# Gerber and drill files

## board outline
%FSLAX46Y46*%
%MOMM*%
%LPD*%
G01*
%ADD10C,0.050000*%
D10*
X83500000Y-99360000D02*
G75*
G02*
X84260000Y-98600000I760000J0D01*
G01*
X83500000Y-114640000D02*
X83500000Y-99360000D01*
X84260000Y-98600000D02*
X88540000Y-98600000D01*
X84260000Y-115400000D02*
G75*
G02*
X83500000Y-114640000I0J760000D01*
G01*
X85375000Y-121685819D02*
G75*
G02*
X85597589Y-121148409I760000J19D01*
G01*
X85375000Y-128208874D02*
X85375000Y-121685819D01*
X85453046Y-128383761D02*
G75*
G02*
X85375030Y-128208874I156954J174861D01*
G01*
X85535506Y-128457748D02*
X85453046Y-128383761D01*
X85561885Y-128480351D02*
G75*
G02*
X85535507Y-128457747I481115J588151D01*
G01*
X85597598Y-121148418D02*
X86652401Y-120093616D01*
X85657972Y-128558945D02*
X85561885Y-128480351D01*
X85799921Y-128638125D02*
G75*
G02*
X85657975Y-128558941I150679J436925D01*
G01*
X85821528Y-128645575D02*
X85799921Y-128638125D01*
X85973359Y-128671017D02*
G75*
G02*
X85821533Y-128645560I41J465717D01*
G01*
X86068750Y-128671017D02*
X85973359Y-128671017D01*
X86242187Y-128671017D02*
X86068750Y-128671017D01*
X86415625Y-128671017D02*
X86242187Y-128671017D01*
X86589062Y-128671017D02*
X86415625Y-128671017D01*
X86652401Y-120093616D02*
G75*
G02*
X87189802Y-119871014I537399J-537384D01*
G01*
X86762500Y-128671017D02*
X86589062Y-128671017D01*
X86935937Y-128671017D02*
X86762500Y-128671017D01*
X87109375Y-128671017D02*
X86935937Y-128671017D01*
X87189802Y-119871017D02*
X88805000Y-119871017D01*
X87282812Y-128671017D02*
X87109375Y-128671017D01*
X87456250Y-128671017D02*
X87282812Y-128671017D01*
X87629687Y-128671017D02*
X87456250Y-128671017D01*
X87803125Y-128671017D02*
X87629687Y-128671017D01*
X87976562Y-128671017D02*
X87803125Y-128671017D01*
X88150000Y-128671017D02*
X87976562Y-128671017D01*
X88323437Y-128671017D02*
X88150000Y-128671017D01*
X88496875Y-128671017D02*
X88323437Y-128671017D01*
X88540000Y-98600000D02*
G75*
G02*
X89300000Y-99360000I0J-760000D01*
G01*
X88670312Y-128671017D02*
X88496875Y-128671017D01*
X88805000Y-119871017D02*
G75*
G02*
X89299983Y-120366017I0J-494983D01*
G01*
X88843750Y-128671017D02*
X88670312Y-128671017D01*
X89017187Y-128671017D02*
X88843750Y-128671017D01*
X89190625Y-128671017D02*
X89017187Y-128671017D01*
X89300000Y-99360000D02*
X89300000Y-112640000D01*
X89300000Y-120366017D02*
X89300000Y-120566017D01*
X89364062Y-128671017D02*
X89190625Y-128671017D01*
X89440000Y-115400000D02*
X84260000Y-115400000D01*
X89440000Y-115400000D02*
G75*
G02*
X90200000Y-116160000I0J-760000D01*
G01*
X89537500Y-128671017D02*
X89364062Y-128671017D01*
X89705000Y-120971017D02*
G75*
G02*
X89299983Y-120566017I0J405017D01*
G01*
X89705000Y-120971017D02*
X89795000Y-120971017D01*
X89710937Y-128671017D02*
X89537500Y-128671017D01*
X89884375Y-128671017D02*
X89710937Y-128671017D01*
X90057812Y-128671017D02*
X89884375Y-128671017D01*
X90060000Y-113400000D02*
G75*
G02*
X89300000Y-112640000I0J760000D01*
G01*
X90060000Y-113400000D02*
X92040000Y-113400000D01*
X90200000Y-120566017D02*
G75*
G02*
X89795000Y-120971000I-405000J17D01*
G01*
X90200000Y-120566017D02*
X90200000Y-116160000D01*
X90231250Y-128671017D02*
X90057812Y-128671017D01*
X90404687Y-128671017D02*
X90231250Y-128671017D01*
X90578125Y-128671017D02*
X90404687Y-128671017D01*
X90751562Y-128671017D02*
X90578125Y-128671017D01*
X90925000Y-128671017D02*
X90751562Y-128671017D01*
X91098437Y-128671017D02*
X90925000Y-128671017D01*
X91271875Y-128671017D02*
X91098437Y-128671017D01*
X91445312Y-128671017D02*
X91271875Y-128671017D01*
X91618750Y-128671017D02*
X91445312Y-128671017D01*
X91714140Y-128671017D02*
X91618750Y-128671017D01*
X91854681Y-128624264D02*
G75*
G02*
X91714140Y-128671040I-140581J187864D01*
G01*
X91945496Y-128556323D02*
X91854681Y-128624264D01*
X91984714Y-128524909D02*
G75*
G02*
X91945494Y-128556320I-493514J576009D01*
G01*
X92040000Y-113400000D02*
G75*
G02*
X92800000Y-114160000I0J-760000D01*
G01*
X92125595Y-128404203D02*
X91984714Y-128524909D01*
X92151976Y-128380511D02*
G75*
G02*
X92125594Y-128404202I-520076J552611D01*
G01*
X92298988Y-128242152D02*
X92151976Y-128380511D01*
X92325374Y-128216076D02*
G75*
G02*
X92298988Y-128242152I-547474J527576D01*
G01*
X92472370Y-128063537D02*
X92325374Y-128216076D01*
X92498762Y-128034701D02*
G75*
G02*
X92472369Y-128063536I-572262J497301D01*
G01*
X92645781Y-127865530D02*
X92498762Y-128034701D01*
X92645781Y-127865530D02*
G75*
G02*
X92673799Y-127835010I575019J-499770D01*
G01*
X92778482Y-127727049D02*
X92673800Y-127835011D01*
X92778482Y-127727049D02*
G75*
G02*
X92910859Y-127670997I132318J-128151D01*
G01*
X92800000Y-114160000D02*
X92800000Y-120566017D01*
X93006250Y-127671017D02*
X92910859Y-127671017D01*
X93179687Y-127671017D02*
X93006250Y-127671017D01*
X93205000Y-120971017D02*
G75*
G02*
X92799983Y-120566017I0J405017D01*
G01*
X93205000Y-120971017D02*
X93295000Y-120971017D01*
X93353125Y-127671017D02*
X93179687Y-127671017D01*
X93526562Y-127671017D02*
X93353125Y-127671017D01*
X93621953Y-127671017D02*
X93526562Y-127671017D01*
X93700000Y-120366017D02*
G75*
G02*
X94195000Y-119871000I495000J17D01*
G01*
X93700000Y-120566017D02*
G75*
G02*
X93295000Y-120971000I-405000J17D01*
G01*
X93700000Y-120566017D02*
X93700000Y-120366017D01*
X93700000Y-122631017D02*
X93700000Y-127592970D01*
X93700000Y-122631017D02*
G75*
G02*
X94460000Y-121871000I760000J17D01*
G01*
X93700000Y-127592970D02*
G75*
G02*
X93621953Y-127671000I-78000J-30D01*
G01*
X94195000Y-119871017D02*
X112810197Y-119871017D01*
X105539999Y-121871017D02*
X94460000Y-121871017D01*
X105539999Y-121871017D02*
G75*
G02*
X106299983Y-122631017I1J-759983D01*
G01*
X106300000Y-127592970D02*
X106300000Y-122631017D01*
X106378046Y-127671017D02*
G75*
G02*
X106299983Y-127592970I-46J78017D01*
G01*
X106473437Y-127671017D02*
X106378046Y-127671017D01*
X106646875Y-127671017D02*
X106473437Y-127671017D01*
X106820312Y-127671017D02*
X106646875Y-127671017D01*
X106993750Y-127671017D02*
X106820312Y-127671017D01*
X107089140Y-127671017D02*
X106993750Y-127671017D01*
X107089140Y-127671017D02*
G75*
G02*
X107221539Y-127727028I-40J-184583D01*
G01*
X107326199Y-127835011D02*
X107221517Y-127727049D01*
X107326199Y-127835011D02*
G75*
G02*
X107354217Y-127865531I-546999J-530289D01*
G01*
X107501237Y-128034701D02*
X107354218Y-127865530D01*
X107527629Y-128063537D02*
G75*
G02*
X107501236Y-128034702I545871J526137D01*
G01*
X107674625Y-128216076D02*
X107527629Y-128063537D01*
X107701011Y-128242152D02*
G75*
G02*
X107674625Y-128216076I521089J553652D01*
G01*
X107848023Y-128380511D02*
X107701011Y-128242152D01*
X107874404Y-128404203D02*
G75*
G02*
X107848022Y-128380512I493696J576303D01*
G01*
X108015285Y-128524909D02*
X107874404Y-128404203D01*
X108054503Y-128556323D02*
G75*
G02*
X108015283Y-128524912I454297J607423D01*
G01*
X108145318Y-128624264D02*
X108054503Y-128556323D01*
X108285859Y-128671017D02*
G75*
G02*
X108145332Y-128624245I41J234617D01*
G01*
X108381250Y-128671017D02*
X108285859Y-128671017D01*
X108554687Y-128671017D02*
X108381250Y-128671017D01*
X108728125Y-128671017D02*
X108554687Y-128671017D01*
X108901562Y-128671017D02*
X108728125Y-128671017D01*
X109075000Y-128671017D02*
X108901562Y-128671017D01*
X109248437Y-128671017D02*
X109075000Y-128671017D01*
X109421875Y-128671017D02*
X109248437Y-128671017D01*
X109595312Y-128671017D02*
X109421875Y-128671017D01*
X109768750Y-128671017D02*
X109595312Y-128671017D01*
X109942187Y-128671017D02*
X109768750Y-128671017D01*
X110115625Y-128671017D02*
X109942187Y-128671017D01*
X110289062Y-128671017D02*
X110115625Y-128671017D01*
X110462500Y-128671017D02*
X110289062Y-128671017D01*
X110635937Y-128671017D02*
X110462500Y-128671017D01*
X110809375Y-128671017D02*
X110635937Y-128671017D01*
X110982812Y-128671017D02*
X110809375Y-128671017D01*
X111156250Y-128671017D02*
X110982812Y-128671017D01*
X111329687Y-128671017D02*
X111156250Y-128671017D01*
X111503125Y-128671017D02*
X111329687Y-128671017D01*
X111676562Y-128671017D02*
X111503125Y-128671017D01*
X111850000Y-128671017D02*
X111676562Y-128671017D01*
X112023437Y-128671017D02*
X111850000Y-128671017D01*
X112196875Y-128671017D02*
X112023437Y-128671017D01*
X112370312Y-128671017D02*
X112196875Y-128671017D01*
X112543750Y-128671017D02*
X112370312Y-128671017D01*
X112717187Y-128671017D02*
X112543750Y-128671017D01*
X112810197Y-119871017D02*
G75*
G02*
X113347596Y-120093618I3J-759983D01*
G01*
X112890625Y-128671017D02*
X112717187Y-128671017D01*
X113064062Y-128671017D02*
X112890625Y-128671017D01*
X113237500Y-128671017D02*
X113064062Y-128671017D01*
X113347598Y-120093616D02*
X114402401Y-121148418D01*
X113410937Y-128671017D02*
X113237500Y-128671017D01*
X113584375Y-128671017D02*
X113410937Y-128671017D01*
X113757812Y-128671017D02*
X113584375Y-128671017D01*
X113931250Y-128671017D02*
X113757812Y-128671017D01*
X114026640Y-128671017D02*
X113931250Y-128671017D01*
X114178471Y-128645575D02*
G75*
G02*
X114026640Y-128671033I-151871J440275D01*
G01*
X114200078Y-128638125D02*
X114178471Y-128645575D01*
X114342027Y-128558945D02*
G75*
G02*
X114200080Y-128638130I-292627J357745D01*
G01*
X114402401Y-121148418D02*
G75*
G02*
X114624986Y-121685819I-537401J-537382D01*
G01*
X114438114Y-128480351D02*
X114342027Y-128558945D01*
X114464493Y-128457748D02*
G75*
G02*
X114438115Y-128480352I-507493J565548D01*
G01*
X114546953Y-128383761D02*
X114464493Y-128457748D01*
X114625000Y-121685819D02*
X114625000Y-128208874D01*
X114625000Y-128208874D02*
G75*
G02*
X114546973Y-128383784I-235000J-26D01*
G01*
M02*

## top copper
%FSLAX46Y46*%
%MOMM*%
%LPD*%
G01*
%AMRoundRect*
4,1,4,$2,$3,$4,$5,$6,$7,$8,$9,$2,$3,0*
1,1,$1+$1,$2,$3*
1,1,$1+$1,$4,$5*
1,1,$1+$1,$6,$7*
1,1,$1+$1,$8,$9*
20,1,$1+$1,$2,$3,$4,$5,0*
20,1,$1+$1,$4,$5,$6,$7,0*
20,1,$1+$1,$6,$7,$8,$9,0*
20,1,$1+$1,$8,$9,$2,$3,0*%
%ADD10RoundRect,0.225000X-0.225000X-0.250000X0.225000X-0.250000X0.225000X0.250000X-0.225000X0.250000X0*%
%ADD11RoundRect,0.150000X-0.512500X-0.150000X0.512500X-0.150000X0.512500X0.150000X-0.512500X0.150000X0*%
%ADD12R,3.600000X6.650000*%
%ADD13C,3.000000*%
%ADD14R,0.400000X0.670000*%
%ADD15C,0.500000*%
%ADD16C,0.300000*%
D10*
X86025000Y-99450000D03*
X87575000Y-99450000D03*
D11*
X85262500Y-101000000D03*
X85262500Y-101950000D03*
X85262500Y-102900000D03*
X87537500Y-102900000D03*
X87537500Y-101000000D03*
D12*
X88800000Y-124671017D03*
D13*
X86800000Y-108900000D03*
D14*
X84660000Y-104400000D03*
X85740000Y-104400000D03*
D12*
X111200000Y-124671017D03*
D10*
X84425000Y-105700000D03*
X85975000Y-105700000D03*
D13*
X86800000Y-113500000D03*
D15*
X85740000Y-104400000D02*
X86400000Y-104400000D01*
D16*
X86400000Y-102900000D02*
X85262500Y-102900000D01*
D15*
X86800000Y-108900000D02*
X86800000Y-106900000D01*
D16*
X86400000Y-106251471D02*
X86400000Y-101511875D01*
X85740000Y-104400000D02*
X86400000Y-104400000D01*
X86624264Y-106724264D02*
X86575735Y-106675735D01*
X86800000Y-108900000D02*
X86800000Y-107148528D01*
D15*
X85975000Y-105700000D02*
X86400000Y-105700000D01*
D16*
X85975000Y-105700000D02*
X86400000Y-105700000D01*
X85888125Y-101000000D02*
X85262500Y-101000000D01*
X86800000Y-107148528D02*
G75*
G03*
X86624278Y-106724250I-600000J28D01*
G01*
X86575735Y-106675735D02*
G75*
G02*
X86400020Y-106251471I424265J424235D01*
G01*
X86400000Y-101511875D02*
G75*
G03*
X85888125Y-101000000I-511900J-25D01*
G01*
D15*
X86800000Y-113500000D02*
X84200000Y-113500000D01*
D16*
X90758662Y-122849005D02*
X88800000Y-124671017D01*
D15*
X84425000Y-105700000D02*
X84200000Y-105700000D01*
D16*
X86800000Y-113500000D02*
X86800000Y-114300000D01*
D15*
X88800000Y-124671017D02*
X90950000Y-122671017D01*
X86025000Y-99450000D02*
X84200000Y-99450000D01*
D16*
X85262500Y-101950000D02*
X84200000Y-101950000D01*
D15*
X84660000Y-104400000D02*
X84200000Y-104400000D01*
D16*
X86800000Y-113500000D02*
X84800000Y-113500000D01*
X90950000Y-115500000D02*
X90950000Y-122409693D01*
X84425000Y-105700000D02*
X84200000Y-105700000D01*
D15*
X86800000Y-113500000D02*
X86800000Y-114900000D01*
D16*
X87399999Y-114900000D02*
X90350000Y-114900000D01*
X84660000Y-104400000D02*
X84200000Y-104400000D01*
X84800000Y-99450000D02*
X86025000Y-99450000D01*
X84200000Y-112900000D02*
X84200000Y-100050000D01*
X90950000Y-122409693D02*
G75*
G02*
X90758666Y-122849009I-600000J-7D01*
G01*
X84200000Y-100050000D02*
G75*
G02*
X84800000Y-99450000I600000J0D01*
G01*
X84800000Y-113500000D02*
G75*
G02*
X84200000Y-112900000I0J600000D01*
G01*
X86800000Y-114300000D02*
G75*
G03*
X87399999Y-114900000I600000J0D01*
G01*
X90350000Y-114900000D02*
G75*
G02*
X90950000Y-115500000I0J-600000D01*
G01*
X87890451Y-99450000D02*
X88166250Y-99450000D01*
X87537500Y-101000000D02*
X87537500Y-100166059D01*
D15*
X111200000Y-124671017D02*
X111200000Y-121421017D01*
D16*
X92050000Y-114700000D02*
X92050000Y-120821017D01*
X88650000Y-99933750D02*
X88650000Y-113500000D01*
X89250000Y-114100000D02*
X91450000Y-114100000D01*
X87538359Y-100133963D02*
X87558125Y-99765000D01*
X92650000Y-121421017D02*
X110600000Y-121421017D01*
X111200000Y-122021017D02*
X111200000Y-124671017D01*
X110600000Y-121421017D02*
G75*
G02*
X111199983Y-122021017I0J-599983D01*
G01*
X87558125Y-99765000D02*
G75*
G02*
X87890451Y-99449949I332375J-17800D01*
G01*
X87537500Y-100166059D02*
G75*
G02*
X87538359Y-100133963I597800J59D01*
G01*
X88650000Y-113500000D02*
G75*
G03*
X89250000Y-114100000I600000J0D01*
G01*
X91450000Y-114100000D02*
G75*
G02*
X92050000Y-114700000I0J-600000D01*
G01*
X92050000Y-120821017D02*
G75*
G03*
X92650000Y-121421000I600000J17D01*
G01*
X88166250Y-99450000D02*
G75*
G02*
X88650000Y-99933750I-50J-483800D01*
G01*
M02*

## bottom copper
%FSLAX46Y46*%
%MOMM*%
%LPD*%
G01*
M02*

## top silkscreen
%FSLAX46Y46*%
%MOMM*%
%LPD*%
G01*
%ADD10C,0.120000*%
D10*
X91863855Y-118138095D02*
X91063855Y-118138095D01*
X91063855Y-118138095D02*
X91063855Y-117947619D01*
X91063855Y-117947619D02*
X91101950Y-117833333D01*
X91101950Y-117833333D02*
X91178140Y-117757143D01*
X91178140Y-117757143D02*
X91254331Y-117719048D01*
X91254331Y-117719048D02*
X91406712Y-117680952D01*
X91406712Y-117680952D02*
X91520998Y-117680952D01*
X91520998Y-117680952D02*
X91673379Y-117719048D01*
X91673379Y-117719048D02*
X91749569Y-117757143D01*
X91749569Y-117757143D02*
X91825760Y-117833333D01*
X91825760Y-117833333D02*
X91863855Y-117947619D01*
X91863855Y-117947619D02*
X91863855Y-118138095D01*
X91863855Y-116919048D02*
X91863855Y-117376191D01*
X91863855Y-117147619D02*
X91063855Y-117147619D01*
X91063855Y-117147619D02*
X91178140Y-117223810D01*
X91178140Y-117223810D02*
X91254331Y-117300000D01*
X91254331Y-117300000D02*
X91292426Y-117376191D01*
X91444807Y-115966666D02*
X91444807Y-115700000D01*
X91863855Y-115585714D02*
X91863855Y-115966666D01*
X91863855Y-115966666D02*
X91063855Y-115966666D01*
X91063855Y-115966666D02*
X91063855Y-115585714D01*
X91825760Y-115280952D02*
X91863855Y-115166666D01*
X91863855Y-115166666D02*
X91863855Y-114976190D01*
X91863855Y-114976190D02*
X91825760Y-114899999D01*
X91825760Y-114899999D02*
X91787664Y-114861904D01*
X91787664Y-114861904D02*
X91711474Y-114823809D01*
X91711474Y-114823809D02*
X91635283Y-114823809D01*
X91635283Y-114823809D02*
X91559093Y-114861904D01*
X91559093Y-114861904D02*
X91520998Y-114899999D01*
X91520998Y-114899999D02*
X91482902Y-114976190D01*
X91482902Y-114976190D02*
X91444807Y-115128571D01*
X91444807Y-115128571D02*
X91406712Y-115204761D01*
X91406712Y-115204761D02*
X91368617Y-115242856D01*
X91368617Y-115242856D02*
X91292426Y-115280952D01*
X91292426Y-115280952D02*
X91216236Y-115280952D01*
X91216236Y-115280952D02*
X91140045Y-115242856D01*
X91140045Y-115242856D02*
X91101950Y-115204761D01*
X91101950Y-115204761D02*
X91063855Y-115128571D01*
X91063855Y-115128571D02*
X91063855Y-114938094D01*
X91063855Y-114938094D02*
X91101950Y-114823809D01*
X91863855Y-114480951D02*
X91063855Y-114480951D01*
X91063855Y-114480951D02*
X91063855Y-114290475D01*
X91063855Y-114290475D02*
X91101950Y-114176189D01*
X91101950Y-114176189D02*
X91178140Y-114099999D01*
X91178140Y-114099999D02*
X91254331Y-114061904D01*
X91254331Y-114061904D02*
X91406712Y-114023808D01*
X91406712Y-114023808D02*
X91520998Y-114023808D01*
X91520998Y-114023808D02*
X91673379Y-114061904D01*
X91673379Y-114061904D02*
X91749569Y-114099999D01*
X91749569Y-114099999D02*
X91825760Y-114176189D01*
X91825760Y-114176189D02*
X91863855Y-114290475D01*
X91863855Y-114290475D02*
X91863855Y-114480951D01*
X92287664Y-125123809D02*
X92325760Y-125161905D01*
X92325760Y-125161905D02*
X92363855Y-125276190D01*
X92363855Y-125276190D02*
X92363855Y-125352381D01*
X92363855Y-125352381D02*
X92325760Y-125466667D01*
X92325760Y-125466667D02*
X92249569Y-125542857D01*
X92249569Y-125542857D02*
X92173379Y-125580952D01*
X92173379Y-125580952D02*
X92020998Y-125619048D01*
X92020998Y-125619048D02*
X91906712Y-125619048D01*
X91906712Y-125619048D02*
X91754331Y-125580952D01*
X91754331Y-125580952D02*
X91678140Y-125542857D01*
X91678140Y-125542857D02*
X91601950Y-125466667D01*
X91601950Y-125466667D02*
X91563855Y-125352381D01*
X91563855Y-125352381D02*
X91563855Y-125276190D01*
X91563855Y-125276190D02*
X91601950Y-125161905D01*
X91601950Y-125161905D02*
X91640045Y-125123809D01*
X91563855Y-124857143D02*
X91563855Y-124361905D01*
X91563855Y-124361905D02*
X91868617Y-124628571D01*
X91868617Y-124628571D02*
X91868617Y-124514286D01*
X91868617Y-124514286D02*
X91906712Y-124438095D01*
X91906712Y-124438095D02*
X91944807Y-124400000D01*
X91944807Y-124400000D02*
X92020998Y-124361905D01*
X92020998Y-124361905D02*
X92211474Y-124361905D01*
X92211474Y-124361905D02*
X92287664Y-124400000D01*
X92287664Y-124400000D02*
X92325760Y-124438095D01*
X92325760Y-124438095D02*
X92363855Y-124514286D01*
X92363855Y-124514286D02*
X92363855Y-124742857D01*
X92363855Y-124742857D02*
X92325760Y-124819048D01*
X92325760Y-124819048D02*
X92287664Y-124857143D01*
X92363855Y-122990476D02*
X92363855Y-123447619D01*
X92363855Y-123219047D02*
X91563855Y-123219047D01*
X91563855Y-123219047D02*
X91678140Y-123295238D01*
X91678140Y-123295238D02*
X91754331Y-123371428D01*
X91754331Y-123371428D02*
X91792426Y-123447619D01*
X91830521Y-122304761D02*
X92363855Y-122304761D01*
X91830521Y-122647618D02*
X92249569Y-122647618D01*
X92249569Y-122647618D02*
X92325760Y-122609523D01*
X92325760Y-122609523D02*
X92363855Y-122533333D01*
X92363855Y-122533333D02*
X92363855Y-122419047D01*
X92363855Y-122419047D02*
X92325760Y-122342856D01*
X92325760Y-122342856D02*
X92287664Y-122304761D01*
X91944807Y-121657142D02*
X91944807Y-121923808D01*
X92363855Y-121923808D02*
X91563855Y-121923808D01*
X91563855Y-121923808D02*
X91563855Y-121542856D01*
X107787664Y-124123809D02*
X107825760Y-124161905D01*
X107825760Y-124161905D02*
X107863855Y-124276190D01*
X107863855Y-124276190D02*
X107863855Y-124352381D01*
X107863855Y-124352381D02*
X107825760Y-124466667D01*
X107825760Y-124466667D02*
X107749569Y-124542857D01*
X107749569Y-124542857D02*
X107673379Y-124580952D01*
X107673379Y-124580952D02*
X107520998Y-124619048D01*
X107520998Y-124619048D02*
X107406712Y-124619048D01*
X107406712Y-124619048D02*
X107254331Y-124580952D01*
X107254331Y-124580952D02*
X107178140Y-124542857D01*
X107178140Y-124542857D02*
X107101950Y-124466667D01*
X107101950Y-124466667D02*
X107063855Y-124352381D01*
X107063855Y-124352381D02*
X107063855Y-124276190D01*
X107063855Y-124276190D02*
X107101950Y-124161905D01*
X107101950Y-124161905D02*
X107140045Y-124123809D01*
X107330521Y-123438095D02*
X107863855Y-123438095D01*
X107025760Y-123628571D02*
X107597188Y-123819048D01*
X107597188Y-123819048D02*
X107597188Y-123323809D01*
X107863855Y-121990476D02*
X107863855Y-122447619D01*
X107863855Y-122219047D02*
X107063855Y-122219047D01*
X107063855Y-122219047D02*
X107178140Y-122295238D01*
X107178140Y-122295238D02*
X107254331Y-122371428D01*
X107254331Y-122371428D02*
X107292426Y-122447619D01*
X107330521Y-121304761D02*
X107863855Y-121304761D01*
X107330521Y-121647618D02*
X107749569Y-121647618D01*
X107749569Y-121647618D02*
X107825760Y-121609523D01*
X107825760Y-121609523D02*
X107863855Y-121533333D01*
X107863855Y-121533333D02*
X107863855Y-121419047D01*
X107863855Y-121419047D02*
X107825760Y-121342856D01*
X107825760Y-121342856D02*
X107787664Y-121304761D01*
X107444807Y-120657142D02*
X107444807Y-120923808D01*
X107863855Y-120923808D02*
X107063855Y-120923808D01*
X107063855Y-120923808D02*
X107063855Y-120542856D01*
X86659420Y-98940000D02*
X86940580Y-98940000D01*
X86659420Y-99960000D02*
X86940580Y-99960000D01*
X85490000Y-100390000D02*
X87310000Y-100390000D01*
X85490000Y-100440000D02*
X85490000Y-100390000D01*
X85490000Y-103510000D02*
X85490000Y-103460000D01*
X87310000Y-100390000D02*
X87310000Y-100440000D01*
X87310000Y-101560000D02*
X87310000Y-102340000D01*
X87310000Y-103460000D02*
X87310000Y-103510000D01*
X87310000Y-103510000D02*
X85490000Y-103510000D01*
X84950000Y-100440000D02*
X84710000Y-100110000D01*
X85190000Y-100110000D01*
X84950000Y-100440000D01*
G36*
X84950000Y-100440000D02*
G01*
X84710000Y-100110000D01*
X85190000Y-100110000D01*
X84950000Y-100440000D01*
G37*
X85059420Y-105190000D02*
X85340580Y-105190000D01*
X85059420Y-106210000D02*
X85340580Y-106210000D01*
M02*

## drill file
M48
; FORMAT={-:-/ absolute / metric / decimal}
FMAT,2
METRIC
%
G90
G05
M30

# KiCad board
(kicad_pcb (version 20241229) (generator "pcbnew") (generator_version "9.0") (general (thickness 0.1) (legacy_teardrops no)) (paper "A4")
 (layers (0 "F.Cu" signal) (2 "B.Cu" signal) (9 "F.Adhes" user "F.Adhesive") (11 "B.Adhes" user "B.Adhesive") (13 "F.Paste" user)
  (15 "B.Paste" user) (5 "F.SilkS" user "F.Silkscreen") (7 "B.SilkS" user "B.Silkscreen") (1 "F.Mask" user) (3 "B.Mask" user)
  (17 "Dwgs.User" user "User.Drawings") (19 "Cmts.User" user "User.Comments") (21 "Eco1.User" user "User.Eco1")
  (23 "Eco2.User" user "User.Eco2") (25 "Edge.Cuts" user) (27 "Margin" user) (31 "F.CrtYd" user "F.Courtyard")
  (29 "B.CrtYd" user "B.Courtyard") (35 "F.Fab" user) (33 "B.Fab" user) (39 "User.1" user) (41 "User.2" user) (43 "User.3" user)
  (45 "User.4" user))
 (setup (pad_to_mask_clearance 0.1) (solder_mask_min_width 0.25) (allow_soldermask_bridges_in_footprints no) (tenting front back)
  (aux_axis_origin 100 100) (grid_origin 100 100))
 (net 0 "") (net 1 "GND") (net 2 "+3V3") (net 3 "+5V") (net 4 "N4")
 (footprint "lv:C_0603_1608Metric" (layer "F.Cu") (at 86.8 99.45)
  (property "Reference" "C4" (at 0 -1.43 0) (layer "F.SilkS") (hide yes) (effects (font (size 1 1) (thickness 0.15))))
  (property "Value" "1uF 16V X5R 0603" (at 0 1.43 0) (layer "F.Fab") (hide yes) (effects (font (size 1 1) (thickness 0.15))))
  (fp_line (start -0.14058 -0.51) (end 0.14058 -0.51) (stroke (width 0.12) (type solid)) (layer "F.SilkS"))
  (fp_line (start -0.14058 0.51) (end 0.14058 0.51) (stroke (width 0.12) (type solid)) (layer "F.SilkS"))
  (pad "1" smd roundrect (at -0.775 0) (size 0.9 0.95) (layers "F.Cu" "F.Mask" "F.Paste") (roundrect_rratio 0.25) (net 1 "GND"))
  (pad "2" smd roundrect (at 0.775 0) (size 0.9 0.95) (layers "F.Cu" "F.Mask" "F.Paste") (roundrect_rratio 0.25) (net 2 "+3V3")))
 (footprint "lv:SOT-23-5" (layer "F.Cu") (at 86.4 101.95)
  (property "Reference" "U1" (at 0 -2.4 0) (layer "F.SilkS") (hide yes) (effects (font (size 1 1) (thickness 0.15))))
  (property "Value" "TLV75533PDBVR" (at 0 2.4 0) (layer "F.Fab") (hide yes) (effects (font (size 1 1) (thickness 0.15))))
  (fp_line (start -0.91 -1.56) (end 0.91 -1.56) (stroke (width 0.12) (type solid)) (layer "F.SilkS"))
  (fp_line (start -0.91 -1.51) (end -0.91 -1.56) (stroke (width 0.12) (type solid)) (layer "F.SilkS"))
  (fp_line (start -0.91 1.56) (end -0.91 1.51) (stroke (width 0.12) (type solid)) (layer "F.SilkS"))
  (fp_line (start 0.91 -1.56) (end 0.91 -1.51) (stroke (width 0.12) (type solid)) (layer "F.SilkS"))
  (fp_line (start 0.91 -0.39) (end 0.91 0.39) (stroke (width 0.12) (type solid)) (layer "F.SilkS"))
  (fp_line (start 0.91 1.51) (end 0.91 1.56) (stroke (width 0.12) (type solid)) (layer "F.SilkS"))
  (fp_line (start 0.91 1.56) (end -0.91 1.56) (stroke (width 0.12) (type solid)) (layer "F.SilkS"))
  (fp_poly (pts (xy -1.45 -1.51) (xy -1.69 -1.84) (xy -1.21 -1.84)) (stroke (width 0.12) (type solid)) (fill yes) (layer "F.SilkS"))
  (pad "1" smd roundrect (at -1.1375 -0.95) (size 1.325 0.6) (layers "F.Cu" "F.Mask" "F.Paste") (roundrect_rratio 0.25) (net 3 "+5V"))
  (pad "2" smd roundrect (at -1.1375 0) (size 1.325 0.6) (layers "F.Cu" "F.Mask" "F.Paste") (roundrect_rratio 0.25) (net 1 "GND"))
  (pad "3" smd roundrect (at -1.1375 0.95) (size 1.325 0.6) (layers "F.Cu" "F.Mask" "F.Paste") (roundrect_rratio 0.25) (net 3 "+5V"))
  (pad "4" smd roundrect (at 1.1375 0.95) (size 1.325 0.6) (layers "F.Cu" "F.Mask" "F.Paste") (roundrect_rratio 0.25) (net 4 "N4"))
  (pad "5" smd roundrect (at 1.1375 -0.95) (size 1.325 0.6) (layers "F.Cu" "F.Mask" "F.Paste") (roundrect_rratio 0.25) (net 2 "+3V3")))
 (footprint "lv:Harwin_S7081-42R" (layer "F.Cu") (at 88.8 124.671017 90)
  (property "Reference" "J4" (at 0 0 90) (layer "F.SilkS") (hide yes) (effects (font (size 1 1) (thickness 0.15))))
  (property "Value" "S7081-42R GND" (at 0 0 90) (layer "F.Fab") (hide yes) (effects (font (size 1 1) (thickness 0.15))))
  (pad "1" smd rect (at 0 0 90) (size 6.65 3.6) (layers "F.Cu" "F.Mask" "F.Paste") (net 1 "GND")))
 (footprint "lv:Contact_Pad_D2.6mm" (layer "F.Cu") (at 86.8 108.9)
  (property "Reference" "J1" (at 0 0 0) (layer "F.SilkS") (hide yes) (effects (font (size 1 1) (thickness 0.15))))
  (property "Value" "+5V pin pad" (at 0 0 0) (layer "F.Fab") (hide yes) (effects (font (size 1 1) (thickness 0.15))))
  (pad "1" smd circle (at 0 0) (size 3 3) (layers "F.Cu" "F.Mask") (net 3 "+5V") (solder_mask_margin -0.2)))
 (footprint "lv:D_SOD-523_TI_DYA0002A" (layer "F.Cu") (at 85.2 104.4)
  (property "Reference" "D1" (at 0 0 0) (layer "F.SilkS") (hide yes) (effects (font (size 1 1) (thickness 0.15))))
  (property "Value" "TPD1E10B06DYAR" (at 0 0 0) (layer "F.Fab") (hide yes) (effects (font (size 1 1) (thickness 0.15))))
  (pad "1" smd rect (at -0.54 0) (size 0.4 0.67) (layers "F.Cu" "F.Mask" "F.Paste") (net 1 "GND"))
  (pad "2" smd rect (at 0.54 0) (size 0.4 0.67) (layers "F.Cu" "F.Mask" "F.Paste") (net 3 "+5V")))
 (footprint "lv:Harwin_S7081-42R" (layer "F.Cu") (at 111.2 124.671017 90)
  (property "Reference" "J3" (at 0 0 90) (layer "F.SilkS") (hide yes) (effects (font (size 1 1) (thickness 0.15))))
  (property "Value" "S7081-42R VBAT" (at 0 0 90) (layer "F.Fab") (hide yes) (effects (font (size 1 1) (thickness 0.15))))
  (pad "1" smd rect (at 0 0 90) (size 6.65 3.6) (layers "F.Cu" "F.Mask" "F.Paste") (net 2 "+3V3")))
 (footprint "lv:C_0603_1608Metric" (layer "F.Cu") (at 85.2 105.7)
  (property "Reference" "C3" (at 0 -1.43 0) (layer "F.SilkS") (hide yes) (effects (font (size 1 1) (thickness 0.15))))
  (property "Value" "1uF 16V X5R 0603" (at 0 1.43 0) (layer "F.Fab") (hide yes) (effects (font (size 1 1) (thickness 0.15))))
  (fp_line (start -0.14058 -0.51) (end 0.14058 -0.51) (stroke (width 0.12) (type solid)) (layer "F.SilkS"))
  (fp_line (start -0.14058 0.51) (end 0.14058 0.51) (stroke (width 0.12) (type solid)) (layer "F.SilkS"))
  (pad "1" smd roundrect (at -0.775 0) (size 0.9 0.95) (layers "F.Cu" "F.Mask" "F.Paste") (roundrect_rratio 0.25) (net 1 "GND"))
  (pad "2" smd roundrect (at 0.775 0) (size 0.9 0.95) (layers "F.Cu" "F.Mask" "F.Paste") (roundrect_rratio 0.25) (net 3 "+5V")))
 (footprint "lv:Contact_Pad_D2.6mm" (layer "F.Cu") (at 86.8 113.5)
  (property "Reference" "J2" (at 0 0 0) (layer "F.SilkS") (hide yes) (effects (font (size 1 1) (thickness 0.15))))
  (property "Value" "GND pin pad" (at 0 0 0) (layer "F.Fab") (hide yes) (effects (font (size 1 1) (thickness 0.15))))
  (pad "1" smd circle (at 0 0) (size 3 3) (layers "F.Cu" "F.Mask") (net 1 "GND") (solder_mask_margin -0.2)))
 (gr_arc (start 83.5 99.36) (mid 83.722598 98.822598) (end 84.26 98.6) (stroke (width 0.05) (type default)) (layer "Edge.Cuts"))
 (gr_line (start 83.5 114.64) (end 83.5 99.36) (stroke (width 0.05) (type default)) (layer "Edge.Cuts"))
 (gr_line (start 84.26 98.6) (end 88.54 98.6) (stroke (width 0.05) (type default)) (layer "Edge.Cuts"))
 (gr_arc (start 84.26 115.4) (mid 83.722598 115.177401) (end 83.5 114.64) (stroke (width 0.05) (type default)) (layer "Edge.Cuts"))
 (gr_arc (start 85.375 121.685819) (mid 85.432851 121.39498) (end 85.597598 121.148418) (stroke (width 0.05) (type default))
  (layer "Edge.Cuts"))
 (gr_line (start 85.375 128.208874) (end 85.375 121.685819) (stroke (width 0.05) (type default)) (layer "Edge.Cuts"))
 (gr_arc (start 85.453046 128.383761) (mid 85.395397 128.30463) (end 85.375 128.208874) (stroke (width 0.05) (type default))
  (layer "Edge.Cuts"))
 (gr_line (start 85.535506 128.457748) (end 85.453046 128.383761) (stroke (width 0.05) (type default)) (layer "Edge.Cuts"))
 (gr_arc (start 85.561885 128.480351) (mid 85.548566 128.4692) (end 85.535506 128.457748) (stroke (width 0.05) (type default))
  (layer "Edge.Cuts"))
 (gr_line (start 85.597598 121.148418) (end 86.652401 120.093616) (stroke (width 0.05) (type default)) (layer "Edge.Cuts"))
 (gr_line (start 85.657972 128.558945) (end 85.561885 128.480351) (stroke (width 0.05) (type default)) (layer "Edge.Cuts"))
 (gr_arc (start 85.799921 128.638125) (mid 85.725438 128.604824) (end 85.657972 128.558945) (stroke (width 0.05) (type default))
  (layer "Edge.Cuts"))
 (gr_line (start 85.821528 128.645575) (end 85.799921 128.638125) (stroke (width 0.05) (type default)) (layer "Edge.Cuts"))
 (gr_arc (start 85.973359 128.671017) (mid 85.896385 128.664613) (end 85.821528 128.645575) (stroke (width 0.05) (type default))
  (layer "Edge.Cuts"))
 (gr_line (start 86.06875 128.671017) (end 85.973359 128.671017) (stroke (width 0.05) (type default)) (layer "Edge.Cuts"))
 (gr_line (start 86.242187 128.671017) (end 86.06875 128.671017) (stroke (width 0.05) (type default)) (layer "Edge.Cuts"))
 (gr_line (start 86.415625 128.671017) (end 86.242187 128.671017) (stroke (width 0.05) (type default)) (layer "Edge.Cuts"))
 (gr_line (start 86.589062 128.671017) (end 86.415625 128.671017) (stroke (width 0.05) (type default)) (layer "Edge.Cuts"))
 (gr_arc (start 86.652401 120.093616) (mid 86.898962 119.928869) (end 87.189802 119.871017) (stroke (width 0.05) (type default))
  (layer "Edge.Cuts"))
 (gr_line (start 86.7625 128.671017) (end 86.589062 128.671017) (stroke (width 0.05) (type default)) (layer "Edge.Cuts"))
 (gr_line (start 86.935937 128.671017) (end 86.7625 128.671017) (stroke (width 0.05) (type default)) (layer "Edge.Cuts"))
 (gr_line (start 87.109375 128.671017) (end 86.935937 128.671017) (stroke (width 0.05) (type default)) (layer "Edge.Cuts"))
 (gr_line (start 87.189802 119.871017) (end 88.805 119.871017) (stroke (width 0.05) (type default)) (layer "Edge.Cuts"))
 (gr_line (start 87.282812 128.671017) (end 87.109375 128.671017) (stroke (width 0.05) (type default)) (layer "Edge.Cuts"))
 (gr_line (start 87.45625 128.671017) (end 87.282812 128.671017) (stroke (width 0.05) (type default)) (layer "Edge.Cuts"))
 (gr_line (start 87.629687 128.671017) (end 87.45625 128.671017) (stroke (width 0.05) (type default)) (layer "Edge.Cuts"))
 (gr_line (start 87.803125 128.671017) (end 87.629687 128.671017) (stroke (width 0.05) (type default)) (layer "Edge.Cuts"))
 (gr_line (start 87.976562 128.671017) (end 87.803125 128.671017) (stroke (width 0.05) (type default)) (layer "Edge.Cuts"))
 (gr_line (start 88.15 128.671017) (end 87.976562 128.671017) (stroke (width 0.05) (type default)) (layer "Edge.Cuts"))
 (gr_line (start 88.323437 128.671017) (end 88.15 128.671017) (stroke (width 0.05) (type default)) (layer "Edge.Cuts"))
 (gr_line (start 88.496875 128.671017) (end 88.323437 128.671017) (stroke (width 0.05) (type default)) (layer "Edge.Cuts"))
 (gr_arc (start 88.54 98.6) (mid 89.077401 98.822598) (end 89.3 99.36) (stroke (width 0.05) (type default)) (layer "Edge.Cuts"))
 (gr_line (start 88.670312 128.671017) (end 88.496875 128.671017) (stroke (width 0.05) (type default)) (layer "Edge.Cuts"))
 (gr_arc (start 88.805 119.871017) (mid 89.155017 120.015999) (end 89.3 120.366017) (stroke (width 0.05) (type default)) (layer "Edge.Cuts"))
 (gr_line (start 88.84375 128.671017) (end 88.670312 128.671017) (stroke (width 0.05) (type default)) (layer "Edge.Cuts"))
 (gr_line (start 89.017187 128.671017) (end 88.84375 128.671017) (stroke (width 0.05) (type default)) (layer "Edge.Cuts"))
 (gr_line (start 89.190625 128.671017) (end 89.017187 128.671017) (stroke (width 0.05) (type default)) (layer "Edge.Cuts"))
 (gr_line (start 89.3 99.36) (end 89.3 112.64) (stroke (width 0.05) (type default)) (layer "Edge.Cuts"))
 (gr_line (start 89.3 120.366017) (end 89.3 120.566017) (stroke (width 0.05) (type default)) (layer "Edge.Cuts"))
 (gr_line (start 89.364062 128.671017) (end 89.190625 128.671017) (stroke (width 0.05) (type default)) (layer "Edge.Cuts"))
 (gr_line (start 89.44 115.4) (end 84.26 115.4) (stroke (width 0.05) (type default)) (layer "Edge.Cuts"))
 (gr_arc (start 89.44 115.4) (mid 89.977401 115.622599) (end 90.2 116.16) (stroke (width 0.05) (type default)) (layer "Edge.Cuts"))
 (gr_line (start 89.5375 128.671017) (end 89.364062 128.671017) (stroke (width 0.05) (type default)) (layer "Edge.Cuts"))
 (gr_arc (start 89.705 120.971017) (mid 89.418616 120.852396) (end 89.3 120.566017) (stroke (width 0.05) (type default)) (layer "Edge.Cuts"))
 (gr_line (start 89.705 120.971017) (end 89.795 120.971017) (stroke (width 0.05) (type default)) (layer "Edge.Cuts"))
 (gr_line (start 89.710937 128.671017) (end 89.5375 128.671017) (stroke (width 0.05) (type default)) (layer "Edge.Cuts"))
 (gr_line (start 89.884375 128.671017) (end 89.710937 128.671017) (stroke (width 0.05) (type default)) (layer "Edge.Cuts"))
 (gr_line (start 90.057812 128.671017) (end 89.884375 128.671017) (stroke (width 0.05) (type default)) (layer "Edge.Cuts"))
 (gr_arc (start 90.06 113.4) (mid 89.522599 113.177401) (end 89.3 112.64) (stroke (width 0.05) (type default)) (layer "Edge.Cuts"))
 (gr_line (start 90.06 113.4) (end 92.04 113.4) (stroke (width 0.05) (type default)) (layer "Edge.Cuts"))
 (gr_arc (start 90.2 120.566017) (mid 90.081372 120.852384) (end 89.795 120.971017) (stroke (width 0.05) (type default)) (layer "Edge.Cuts"))
 (gr_line (start 90.2 120.566017) (end 90.2 116.16) (stroke (width 0.05) (type default)) (layer "Edge.Cuts"))
 (gr_line (start 90.23125 128.671017) (end 90.057812 128.671017) (stroke (width 0.05) (type default)) (layer "Edge.Cuts"))
 (gr_line (start 90.404687 128.671017) (end 90.23125 128.671017) (stroke (width 0.05) (type default)) (layer "Edge.Cuts"))
 (gr_line (start 90.578125 128.671017) (end 90.404687 128.671017) (stroke (width 0.05) (type default)) (layer "Edge.Cuts"))
 (gr_line (start 90.751562 128.671017) (end 90.578125 128.671017) (stroke (width 0.05) (type default)) (layer "Edge.Cuts"))
 (gr_line (start 90.925 128.671017) (end 90.751562 128.671017) (stroke (width 0.05) (type default)) (layer "Edge.Cuts"))
 (gr_line (start 91.098437 128.671017) (end 90.925 128.671017) (stroke (width 0.05) (type default)) (layer "Edge.Cuts"))
 (gr_line (start 91.271875 128.671017) (end 91.098437 128.671017) (stroke (width 0.05) (type default)) (layer "Edge.Cuts"))
 (gr_line (start 91.445312 128.671017) (end 91.271875 128.671017) (stroke (width 0.05) (type default)) (layer "Edge.Cuts"))
 (gr_line (start 91.61875 128.671017) (end 91.445312 128.671017) (stroke (width 0.05) (type default)) (layer "Edge.Cuts"))
 (gr_line (start 91.71414 128.671017) (end 91.61875 128.671017) (stroke (width 0.05) (type default)) (layer "Edge.Cuts"))
 (gr_arc (start 91.854681 128.624264) (mid 91.788197 128.659022) (end 91.71414 128.671017) (stroke (width 0.05) (type default))
  (layer "Edge.Cuts"))
 (gr_line (start 91.945496 128.556323) (end 91.854681 128.624264) (stroke (width 0.05) (type default)) (layer "Edge.Cuts"))
 (gr_arc (start 91.984714 128.524909) (mid 91.965365 128.540941) (end 91.945496 128.556323) (stroke (width 0.05) (type default))
  (layer "Edge.Cuts"))
 (gr_arc (start 92.04 113.4) (mid 92.577401 113.622598) (end 92.8 114.16) (stroke (width 0.05) (type default)) (layer "Edge.Cuts"))
 (gr_line (start 92.125595 128.404203) (end 91.984714 128.524909) (stroke (width 0.05) (type default)) (layer "Edge.Cuts"))
 (gr_arc (start 92.151976 128.380511) (mid 92.138924 128.392511) (end 92.125595 128.404203) (stroke (width 0.05) (type default))
  (layer "Edge.Cuts"))
 (gr_line (start 92.298988 128.242152) (end 92.151976 128.380511) (stroke (width 0.05) (type default)) (layer "Edge.Cuts"))
 (gr_arc (start 92.325374 128.216076) (mid 92.31234 128.229275) (end 92.298988 128.242152) (stroke (width 0.05) (type default))
  (layer "Edge.Cuts"))
 (gr_line (start 92.47237 128.063537) (end 92.325374 128.216076) (stroke (width 0.05) (type default)) (layer "Edge.Cuts"))
 (gr_arc (start 92.498762 128.034701) (mid 92.485752 128.049289) (end 92.47237 128.063537) (stroke (width 0.05) (type default))
  (layer "Edge.Cuts"))
 (gr_line (start 92.645781 127.86553) (end 92.498762 128.034701) (stroke (width 0.05) (type default)) (layer "Edge.Cuts"))
 (gr_arc (start 92.645781 127.86553) (mid 92.659583 127.85008) (end 92.6738 127.835011) (stroke (width 0.05) (type default))
  (layer "Edge.Cuts"))
 (gr_line (start 92.778482 127.727049) (end 92.6738 127.835011) (stroke (width 0.05) (type default)) (layer "Edge.Cuts"))
 (gr_arc (start 92.778482 127.727049) (mid 92.838983 127.685587) (end 92.910859 127.671017) (stroke (width 0.05) (type default))
  (layer "Edge.Cuts"))
 (gr_line (start 92.8 114.16) (end 92.8 120.566017) (stroke (width 0.05) (type default)) (layer "Edge.Cuts"))
 (gr_line (start 93.00625 127.671017) (end 92.910859 127.671017) (stroke (width 0.05) (type default)) (layer "Edge.Cuts"))
 (gr_line (start 93.179687 127.671017) (end 93.00625 127.671017) (stroke (width 0.05) (type default)) (layer "Edge.Cuts"))
 (gr_arc (start 93.205 120.971017) (mid 92.918616 120.852396) (end 92.8 120.566017) (stroke (width 0.05) (type default)) (layer "Edge.Cuts"))
 (gr_line (start 93.205 120.971017) (end 93.295 120.971017) (stroke (width 0.05) (type default)) (layer "Edge.Cuts"))
 (gr_line (start 93.353125 127.671017) (end 93.179687 127.671017) (stroke (width 0.05) (type default)) (layer "Edge.Cuts"))
 (gr_line (start 93.526562 127.671017) (end 93.353125 127.671017) (stroke (width 0.05) (type default)) (layer "Edge.Cuts"))
 (gr_line (start 93.621953 127.671017) (end 93.526562 127.671017) (stroke (width 0.05) (type default)) (layer "Edge.Cuts"))
 (gr_arc (start 93.7 120.366017) (mid 93.844982 120.015999) (end 94.195 119.871017) (stroke (width 0.05) (type default)) (layer "Edge.Cuts"))
 (gr_arc (start 93.7 120.566017) (mid 93.581372 120.852384) (end 93.295 120.971017) (stroke (width 0.05) (type default)) (layer "Edge.Cuts"))
 (gr_line (start 93.7 120.566017) (end 93.7 120.366017) (stroke (width 0.05) (type default)) (layer "Edge.Cuts"))
 (gr_line (start 93.7 122.631017) (end 93.7 127.59297) (stroke (width 0.05) (type default)) (layer "Edge.Cuts"))
 (gr_arc (start 93.7 122.631017) (mid 93.922593 122.093605) (end 94.46 121.871017) (stroke (width 0.05) (type default)) (layer "Edge.Cuts"))
 (gr_arc (start 93.7 127.59297) (mid 93.67714 127.648158) (end 93.621953 127.671017) (stroke (width 0.05) (type default))
  (layer "Edge.Cuts"))
 (gr_line (start 94.195 119.871017) (end 112.810197 119.871017) (stroke (width 0.05) (type default)) (layer "Edge.Cuts"))
 (gr_line (start 105.539999 121.871017) (end 94.46 121.871017) (stroke (width 0.05) (type default)) (layer "Edge.Cuts"))
 (gr_arc (start 105.539999 121.871017) (mid 106.077395 122.093617) (end 106.3 122.631017) (stroke (width 0.05) (type default))
  (layer "Edge.Cuts"))
 (gr_line (start 106.3 127.59297) (end 106.3 122.631017) (stroke (width 0.05) (type default)) (layer "Edge.Cuts"))
 (gr_arc (start 106.378046 127.671017) (mid 106.322859 127.648158) (end 106.3 127.59297) (stroke (width 0.05) (type default))
  (layer "Edge.Cuts"))
 (gr_line (start 106.473437 127.671017) (end 106.378046 127.671017) (stroke (width 0.05) (type default)) (layer "Edge.Cuts"))
 (gr_line (start 106.646875 127.671017) (end 106.473437 127.671017) (stroke (width 0.05) (type default)) (layer "Edge.Cuts"))
 (gr_line (start 106.820312 127.671017) (end 106.646875 127.671017) (stroke (width 0.05) (type default)) (layer "Edge.Cuts"))
 (gr_line (start 106.99375 127.671017) (end 106.820312 127.671017) (stroke (width 0.05) (type default)) (layer "Edge.Cuts"))
 (gr_line (start 107.08914 127.671017) (end 106.99375 127.671017) (stroke (width 0.05) (type default)) (layer "Edge.Cuts"))
 (gr_arc (start 107.08914 127.671017) (mid 107.161005 127.685615) (end 107.221517 127.727049) (stroke (width 0.05) (type default))
  (layer "Edge.Cuts"))
 (gr_line (start 107.326199 127.835011) (end 107.221517 127.727049) (stroke (width 0.05) (type default)) (layer "Edge.Cuts"))
 (gr_arc (start 107.326199 127.835011) (mid 107.340416 127.85008) (end 107.354218 127.86553) (stroke (width 0.05) (type default))
  (layer "Edge.Cuts"))
 (gr_line (start 107.501237 128.034701) (end 107.354218 127.86553) (stroke (width 0.05) (type default)) (layer "Edge.Cuts"))
 (gr_arc (start 107.527629 128.063537) (mid 107.514247 128.049289) (end 107.501237 128.034701) (stroke (width 0.05) (type default))
  (layer "Edge.Cuts"))
 (gr_line (start 107.674625 128.216076) (end 107.527629 128.063537) (stroke (width 0.05) (type default)) (layer "Edge.Cuts"))
 (gr_arc (start 107.701011 128.242152) (mid 107.687659 128.229275) (end 107.674625 128.216076) (stroke (width 0.05) (type default))
  (layer "Edge.Cuts"))
 (gr_line (start 107.848023 128.380511) (end 107.701011 128.242152) (stroke (width 0.05) (type default)) (layer "Edge.Cuts"))
 (gr_arc (start 107.874404 128.404203) (mid 107.861075 128.392511) (end 107.848023 128.380511) (stroke (width 0.05) (type default))
  (layer "Edge.Cuts"))
 (gr_line (start 108.015285 128.524909) (end 107.874404 128.404203) (stroke (width 0.05) (type default)) (layer "Edge.Cuts"))
 (gr_arc (start 108.054503 128.556323) (mid 108.034634 128.540941) (end 108.015285 128.524909) (stroke (width 0.05) (type default))
  (layer "Edge.Cuts"))
 (gr_line (start 108.145318 128.624264) (end 108.054503 128.556323) (stroke (width 0.05) (type default)) (layer "Edge.Cuts"))
 (gr_arc (start 108.285859 128.671017) (mid 108.211802 128.659022) (end 108.145318 128.624264) (stroke (width 0.05) (type default))
  (layer "Edge.Cuts"))
 (gr_line (start 108.38125 128.671017) (end 108.285859 128.671017) (stroke (width 0.05) (type default)) (layer "Edge.Cuts"))
 (gr_line (start 108.554687 128.671017) (end 108.38125 128.671017) (stroke (width 0.05) (type default)) (layer "Edge.Cuts"))
 (gr_line (start 108.728125 128.671017) (end 108.554687 128.671017) (stroke (width 0.05) (type default)) (layer "Edge.Cuts"))
 (gr_line (start 108.901562 128.671017) (end 108.728125 128.671017) (stroke (width 0.05) (type default)) (layer "Edge.Cuts"))
 (gr_line (start 109.075 128.671017) (end 108.901562 128.671017) (stroke (width 0.05) (type default)) (layer "Edge.Cuts"))
 (gr_line (start 109.248437 128.671017) (end 109.075 128.671017) (stroke (width 0.05) (type default)) (layer "Edge.Cuts"))
 (gr_line (start 109.421875 128.671017) (end 109.248437 128.671017) (stroke (width 0.05) (type default)) (layer "Edge.Cuts"))
 (gr_line (start 109.595312 128.671017) (end 109.421875 128.671017) (stroke (width 0.05) (type default)) (layer "Edge.Cuts"))
 (gr_line (start 109.76875 128.671017) (end 109.595312 128.671017) (stroke (width 0.05) (type default)) (layer "Edge.Cuts"))
 (gr_line (start 109.942187 128.671017) (end 109.76875 128.671017) (stroke (width 0.05) (type default)) (layer "Edge.Cuts"))
 (gr_line (start 110.115625 128.671017) (end 109.942187 128.671017) (stroke (width 0.05) (type default)) (layer "Edge.Cuts"))
 (gr_line (start 110.289062 128.671017) (end 110.115625 128.671017) (stroke (width 0.05) (type default)) (layer "Edge.Cuts"))
 (gr_line (start 110.4625 128.671017) (end 110.289062 128.671017) (stroke (width 0.05) (type default)) (layer "Edge.Cuts"))
 (gr_line (start 110.635937 128.671017) (end 110.4625 128.671017) (stroke (width 0.05) (type default)) (layer "Edge.Cuts"))
 (gr_line (start 110.809375 128.671017) (end 110.635937 128.671017) (stroke (width 0.05) (type default)) (layer "Edge.Cuts"))
 (gr_line (start 110.982812 128.671017) (end 110.809375 128.671017) (stroke (width 0.05) (type default)) (layer "Edge.Cuts"))
 (gr_line (start 111.15625 128.671017) (end 110.982812 128.671017) (stroke (width 0.05) (type default)) (layer "Edge.Cuts"))
 (gr_line (start 111.329687 128.671017) (end 111.15625 128.671017) (stroke (width 0.05) (type default)) (layer "Edge.Cuts"))
 (gr_line (start 111.503125 128.671017) (end 111.329687 128.671017) (stroke (width 0.05) (type default)) (layer "Edge.Cuts"))
 (gr_line (start 111.676562 128.671017) (end 111.503125 128.671017) (stroke (width 0.05) (type default)) (layer "Edge.Cuts"))
 (gr_line (start 111.85 128.671017) (end 111.676562 128.671017) (stroke (width 0.05) (type default)) (layer "Edge.Cuts"))
 (gr_line (start 112.023437 128.671017) (end 111.85 128.671017) (stroke (width 0.05) (type default)) (layer "Edge.Cuts"))
 (gr_line (start 112.196875 128.671017) (end 112.023437 128.671017) (stroke (width 0.05) (type default)) (layer "Edge.Cuts"))
 (gr_line (start 112.370312 128.671017) (end 112.196875 128.671017) (stroke (width 0.05) (type default)) (layer "Edge.Cuts"))
 (gr_line (start 112.54375 128.671017) (end 112.370312 128.671017) (stroke (width 0.05) (type default)) (layer "Edge.Cuts"))
 (gr_line (start 112.717187 128.671017) (end 112.54375 128.671017) (stroke (width 0.05) (type default)) (layer "Edge.Cuts"))
 (gr_arc (start 112.810197 119.871017) (mid 113.101037 119.928869) (end 113.347598 120.093616) (stroke (width 0.05) (type default))
  (layer "Edge.Cuts"))
 (gr_line (start 112.890625 128.671017) (end 112.717187 128.671017) (stroke (width 0.05) (type default)) (layer "Edge.Cuts"))
 (gr_line (start 113.064062 128.671017) (end 112.890625 128.671017) (stroke (width 0.05) (type default)) (layer "Edge.Cuts"))
 (gr_line (start 113.2375 128.671017) (end 113.064062 128.671017) (stroke (width 0.05) (type default)) (layer "Edge.Cuts"))
 (gr_line (start 113.347598 120.093616) (end 114.402401 121.148418) (stroke (width 0.05) (type default)) (layer "Edge.Cuts"))
 (gr_line (start 113.410937 128.671017) (end 113.2375 128.671017) (stroke (width 0.05) (type default)) (layer "Edge.Cuts"))
 (gr_line (start 113.584375 128.671017) (end 113.410937 128.671017) (stroke (width 0.05) (type default)) (layer "Edge.Cuts"))
 (gr_line (start 113.757812 128.671017) (end 113.584375 128.671017) (stroke (width 0.05) (type default)) (layer "Edge.Cuts"))
 (gr_line (start 113.93125 128.671017) (end 113.757812 128.671017) (stroke (width 0.05) (type default)) (layer "Edge.Cuts"))
 (gr_line (start 114.02664 128.671017) (end 113.93125 128.671017) (stroke (width 0.05) (type default)) (layer "Edge.Cuts"))
 (gr_arc (start 114.178471 128.645575) (mid 114.103614 128.664613) (end 114.02664 128.671017) (stroke (width 0.05) (type default))
  (layer "Edge.Cuts"))
 (gr_line (start 114.200078 128.638125) (end 114.178471 128.645575) (stroke (width 0.05) (type default)) (layer "Edge.Cuts"))
 (gr_arc (start 114.342027 128.558945) (mid 114.274561 128.604824) (end 114.200078 128.638125) (stroke (width 0.05) (type default))
  (layer "Edge.Cuts"))
 (gr_arc (start 114.402401 121.148418) (mid 114.567148 121.39498) (end 114.625 121.685819) (stroke (width 0.05) (type default))
  (layer "Edge.Cuts"))
 (gr_line (start 114.438114 128.480351) (end 114.342027 128.558945) (stroke (width 0.05) (type default)) (layer "Edge.Cuts"))
 (gr_arc (start 114.464493 128.457748) (mid 114.451433 128.4692) (end 114.438114 128.480351) (stroke (width 0.05) (type default))
  (layer "Edge.Cuts"))
 (gr_line (start 114.546953 128.383761) (end 114.464493 128.457748) (stroke (width 0.05) (type default)) (layer "Edge.Cuts"))
 (gr_line (start 114.625 121.685819) (end 114.625 128.208874) (stroke (width 0.05) (type default)) (layer "Edge.Cuts"))
 (gr_arc (start 114.625 128.208874) (mid 114.604602 128.30463) (end 114.546953 128.383761) (stroke (width 0.05) (type default))
  (layer "Edge.Cuts"))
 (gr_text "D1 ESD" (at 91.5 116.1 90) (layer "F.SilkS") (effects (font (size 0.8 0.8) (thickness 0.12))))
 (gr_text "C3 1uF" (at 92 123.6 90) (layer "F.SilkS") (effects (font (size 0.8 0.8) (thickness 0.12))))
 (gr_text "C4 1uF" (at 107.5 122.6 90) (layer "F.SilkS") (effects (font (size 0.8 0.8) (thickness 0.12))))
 (segment (start 85.74 104.4) (end 86.4 104.4) (width 0.5) (layer "F.Cu") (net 3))
 (segment (start 86.4 102.9) (end 85.2625 102.9) (width 0.3) (layer "F.Cu") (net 3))
 (segment (start 86.8 108.9) (end 86.8 106.9) (width 0.5) (layer "F.Cu") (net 3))
 (segment (start 86.4 106.251471) (end 86.4 101.511875) (width 0.3) (layer "F.Cu") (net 3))
 (segment (start 85.74 104.4) (end 86.4 104.4) (width 0.3) (layer "F.Cu") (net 3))
 (segment (start 86.624264 106.724264) (end 86.575735 106.675735) (width 0.3) (layer "F.Cu") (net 3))
 (segment (start 86.8 108.9) (end 86.8 107.148528) (width 0.3) (layer "F.Cu") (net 3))
 (segment (start 85.975 105.7) (end 86.4 105.7) (width 0.5) (layer "F.Cu") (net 3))
 (segment (start 85.975 105.7) (end 86.4 105.7) (width 0.3) (layer "F.Cu") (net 3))
 (segment (start 85.888125 101) (end 85.2625 101) (width 0.3) (layer "F.Cu") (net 3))
 (arc (start 86.8 107.148528) (mid 86.754327 106.918918) (end 86.624264 106.724264) (width 0.3) (layer "F.Cu") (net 3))
 (arc (start 86.575735 106.675735) (mid 86.445672 106.481081) (end 86.4 106.251471) (width 0.3) (layer "F.Cu") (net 3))
 (arc (start 86.4 101.511875) (mid 86.250075 101.149924) (end 85.888125 101) (width 0.3) (layer "F.Cu") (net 3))
 (segment (start 86.8 113.5) (end 84.2 113.5) (width 0.5) (layer "F.Cu") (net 1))
 (segment (start 90.758662 122.849005) (end 88.8 124.671017) (width 0.3) (layer "F.Cu") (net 1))
 (segment (start 84.425 105.7) (end 84.2 105.7) (width 0.5) (layer "F.Cu") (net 1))
 (segment (start 86.8 113.5) (end 86.8 114.3) (width 0.3) (layer "F.Cu") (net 1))
 (segment (start 88.8 124.671017) (end 90.95 122.671017) (width 0.5) (layer "F.Cu") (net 1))
 (segment (start 86.025 99.45) (end 84.2 99.45) (width 0.5) (layer "F.Cu") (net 1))
 (segment (start 85.2625 101.95) (end 84.2 101.95) (width 0.3) (layer "F.Cu") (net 1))
 (segment (start 84.66 104.4) (end 84.2 104.4) (width 0.5) (layer "F.Cu") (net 1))
 (segment (start 86.8 113.5) (end 84.8 113.5) (width 0.3) (layer "F.Cu") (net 1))
 (segment (start 90.95 115.5) (end 90.95 122.409693) (width 0.3) (layer "F.Cu") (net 1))
 (segment (start 84.425 105.7) (end 84.2 105.7) (width 0.3) (layer "F.Cu") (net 1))
 (segment (start 86.8 113.5) (end 86.8 114.9) (width 0.5) (layer "F.Cu") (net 1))
 (segment (start 87.399999 114.9) (end 90.35 114.9) (width 0.3) (layer "F.Cu") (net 1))
 (segment (start 84.66 104.4) (end 84.2 104.4) (width 0.3) (layer "F.Cu") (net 1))
 (segment (start 84.8 99.45) (end 86.025 99.45) (width 0.3) (layer "F.Cu") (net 1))
 (segment (start 84.2 112.9) (end 84.2 100.05) (width 0.3) (layer "F.Cu") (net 1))
 (arc (start 90.95 122.409693) (mid 90.900089 122.649279) (end 90.758662 122.849005) (width 0.3) (layer "F.Cu") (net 1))
 (arc (start 84.2 100.05) (mid 84.375735 99.625735) (end 84.8 99.45) (width 0.3) (layer "F.Cu") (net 1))
 (arc (start 84.8 113.5) (mid 84.375735 113.324264) (end 84.2 112.9) (width 0.3) (layer "F.Cu") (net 1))
 (arc (start 86.8 114.3) (mid 86.975735 114.724264) (end 87.399999 114.9) (width 0.3) (layer "F.Cu") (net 1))
 (arc (start 90.35 114.9) (mid 90.774264 115.075735) (end 90.95 115.5) (width 0.3) (layer "F.Cu") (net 1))
 (segment (start 87.890451 99.45) (end 88.16625 99.45) (width 0.3) (layer "F.Cu") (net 2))
 (segment (start 87.5375 101) (end 87.5375 100.166059) (width 0.3) (layer "F.Cu") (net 2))
 (segment (start 111.2 124.671017) (end 111.2 121.421017) (width 0.5) (layer "F.Cu") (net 2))
 (segment (start 92.05 114.7) (end 92.05 120.821017) (width 0.3) (layer "F.Cu") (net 2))
 (segment (start 88.65 99.93375) (end 88.65 113.5) (width 0.3) (layer "F.Cu") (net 2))
 (segment (start 89.25 114.1) (end 91.45 114.1) (width 0.3) (layer "F.Cu") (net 2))
 (segment (start 87.538359 100.133963) (end 87.558125 99.765) (width 0.3) (layer "F.Cu") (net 2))
 (segment (start 92.65 121.421017) (end 110.6 121.421017) (width 0.3) (layer "F.Cu") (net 2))
 (segment (start 111.2 122.021017) (end 111.2 124.671017) (width 0.3) (layer "F.Cu") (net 2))
 (arc (start 110.6 121.421017) (mid 111.024264 121.596753) (end 111.2 122.021017) (width 0.3) (layer "F.Cu") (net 2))
 (arc (start 87.558125 99.765) (mid 87.661505 99.541263) (end 87.890451 99.45) (width 0.3) (layer "F.Cu") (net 2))
 (arc (start 87.5375 100.166059) (mid 87.537714 100.150005) (end 87.538359 100.133963) (width 0.3) (layer "F.Cu") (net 2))
 (arc (start 88.65 113.5) (mid 88.825735 113.924264) (end 89.25 114.1) (width 0.3) (layer "F.Cu") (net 2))
 (arc (start 91.45 114.1) (mid 91.874264 114.275735) (end 92.05 114.7) (width 0.3) (layer "F.Cu") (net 2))
 (arc (start 92.05 120.821017) (mid 92.225735 121.245281) (end 92.65 121.421017) (width 0.3) (layer "F.Cu") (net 2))
 (arc (start 88.16625 99.45) (mid 88.508312 99.591687) (end 88.65 99.93375) (width 0.3) (layer "F.Cu") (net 2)))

